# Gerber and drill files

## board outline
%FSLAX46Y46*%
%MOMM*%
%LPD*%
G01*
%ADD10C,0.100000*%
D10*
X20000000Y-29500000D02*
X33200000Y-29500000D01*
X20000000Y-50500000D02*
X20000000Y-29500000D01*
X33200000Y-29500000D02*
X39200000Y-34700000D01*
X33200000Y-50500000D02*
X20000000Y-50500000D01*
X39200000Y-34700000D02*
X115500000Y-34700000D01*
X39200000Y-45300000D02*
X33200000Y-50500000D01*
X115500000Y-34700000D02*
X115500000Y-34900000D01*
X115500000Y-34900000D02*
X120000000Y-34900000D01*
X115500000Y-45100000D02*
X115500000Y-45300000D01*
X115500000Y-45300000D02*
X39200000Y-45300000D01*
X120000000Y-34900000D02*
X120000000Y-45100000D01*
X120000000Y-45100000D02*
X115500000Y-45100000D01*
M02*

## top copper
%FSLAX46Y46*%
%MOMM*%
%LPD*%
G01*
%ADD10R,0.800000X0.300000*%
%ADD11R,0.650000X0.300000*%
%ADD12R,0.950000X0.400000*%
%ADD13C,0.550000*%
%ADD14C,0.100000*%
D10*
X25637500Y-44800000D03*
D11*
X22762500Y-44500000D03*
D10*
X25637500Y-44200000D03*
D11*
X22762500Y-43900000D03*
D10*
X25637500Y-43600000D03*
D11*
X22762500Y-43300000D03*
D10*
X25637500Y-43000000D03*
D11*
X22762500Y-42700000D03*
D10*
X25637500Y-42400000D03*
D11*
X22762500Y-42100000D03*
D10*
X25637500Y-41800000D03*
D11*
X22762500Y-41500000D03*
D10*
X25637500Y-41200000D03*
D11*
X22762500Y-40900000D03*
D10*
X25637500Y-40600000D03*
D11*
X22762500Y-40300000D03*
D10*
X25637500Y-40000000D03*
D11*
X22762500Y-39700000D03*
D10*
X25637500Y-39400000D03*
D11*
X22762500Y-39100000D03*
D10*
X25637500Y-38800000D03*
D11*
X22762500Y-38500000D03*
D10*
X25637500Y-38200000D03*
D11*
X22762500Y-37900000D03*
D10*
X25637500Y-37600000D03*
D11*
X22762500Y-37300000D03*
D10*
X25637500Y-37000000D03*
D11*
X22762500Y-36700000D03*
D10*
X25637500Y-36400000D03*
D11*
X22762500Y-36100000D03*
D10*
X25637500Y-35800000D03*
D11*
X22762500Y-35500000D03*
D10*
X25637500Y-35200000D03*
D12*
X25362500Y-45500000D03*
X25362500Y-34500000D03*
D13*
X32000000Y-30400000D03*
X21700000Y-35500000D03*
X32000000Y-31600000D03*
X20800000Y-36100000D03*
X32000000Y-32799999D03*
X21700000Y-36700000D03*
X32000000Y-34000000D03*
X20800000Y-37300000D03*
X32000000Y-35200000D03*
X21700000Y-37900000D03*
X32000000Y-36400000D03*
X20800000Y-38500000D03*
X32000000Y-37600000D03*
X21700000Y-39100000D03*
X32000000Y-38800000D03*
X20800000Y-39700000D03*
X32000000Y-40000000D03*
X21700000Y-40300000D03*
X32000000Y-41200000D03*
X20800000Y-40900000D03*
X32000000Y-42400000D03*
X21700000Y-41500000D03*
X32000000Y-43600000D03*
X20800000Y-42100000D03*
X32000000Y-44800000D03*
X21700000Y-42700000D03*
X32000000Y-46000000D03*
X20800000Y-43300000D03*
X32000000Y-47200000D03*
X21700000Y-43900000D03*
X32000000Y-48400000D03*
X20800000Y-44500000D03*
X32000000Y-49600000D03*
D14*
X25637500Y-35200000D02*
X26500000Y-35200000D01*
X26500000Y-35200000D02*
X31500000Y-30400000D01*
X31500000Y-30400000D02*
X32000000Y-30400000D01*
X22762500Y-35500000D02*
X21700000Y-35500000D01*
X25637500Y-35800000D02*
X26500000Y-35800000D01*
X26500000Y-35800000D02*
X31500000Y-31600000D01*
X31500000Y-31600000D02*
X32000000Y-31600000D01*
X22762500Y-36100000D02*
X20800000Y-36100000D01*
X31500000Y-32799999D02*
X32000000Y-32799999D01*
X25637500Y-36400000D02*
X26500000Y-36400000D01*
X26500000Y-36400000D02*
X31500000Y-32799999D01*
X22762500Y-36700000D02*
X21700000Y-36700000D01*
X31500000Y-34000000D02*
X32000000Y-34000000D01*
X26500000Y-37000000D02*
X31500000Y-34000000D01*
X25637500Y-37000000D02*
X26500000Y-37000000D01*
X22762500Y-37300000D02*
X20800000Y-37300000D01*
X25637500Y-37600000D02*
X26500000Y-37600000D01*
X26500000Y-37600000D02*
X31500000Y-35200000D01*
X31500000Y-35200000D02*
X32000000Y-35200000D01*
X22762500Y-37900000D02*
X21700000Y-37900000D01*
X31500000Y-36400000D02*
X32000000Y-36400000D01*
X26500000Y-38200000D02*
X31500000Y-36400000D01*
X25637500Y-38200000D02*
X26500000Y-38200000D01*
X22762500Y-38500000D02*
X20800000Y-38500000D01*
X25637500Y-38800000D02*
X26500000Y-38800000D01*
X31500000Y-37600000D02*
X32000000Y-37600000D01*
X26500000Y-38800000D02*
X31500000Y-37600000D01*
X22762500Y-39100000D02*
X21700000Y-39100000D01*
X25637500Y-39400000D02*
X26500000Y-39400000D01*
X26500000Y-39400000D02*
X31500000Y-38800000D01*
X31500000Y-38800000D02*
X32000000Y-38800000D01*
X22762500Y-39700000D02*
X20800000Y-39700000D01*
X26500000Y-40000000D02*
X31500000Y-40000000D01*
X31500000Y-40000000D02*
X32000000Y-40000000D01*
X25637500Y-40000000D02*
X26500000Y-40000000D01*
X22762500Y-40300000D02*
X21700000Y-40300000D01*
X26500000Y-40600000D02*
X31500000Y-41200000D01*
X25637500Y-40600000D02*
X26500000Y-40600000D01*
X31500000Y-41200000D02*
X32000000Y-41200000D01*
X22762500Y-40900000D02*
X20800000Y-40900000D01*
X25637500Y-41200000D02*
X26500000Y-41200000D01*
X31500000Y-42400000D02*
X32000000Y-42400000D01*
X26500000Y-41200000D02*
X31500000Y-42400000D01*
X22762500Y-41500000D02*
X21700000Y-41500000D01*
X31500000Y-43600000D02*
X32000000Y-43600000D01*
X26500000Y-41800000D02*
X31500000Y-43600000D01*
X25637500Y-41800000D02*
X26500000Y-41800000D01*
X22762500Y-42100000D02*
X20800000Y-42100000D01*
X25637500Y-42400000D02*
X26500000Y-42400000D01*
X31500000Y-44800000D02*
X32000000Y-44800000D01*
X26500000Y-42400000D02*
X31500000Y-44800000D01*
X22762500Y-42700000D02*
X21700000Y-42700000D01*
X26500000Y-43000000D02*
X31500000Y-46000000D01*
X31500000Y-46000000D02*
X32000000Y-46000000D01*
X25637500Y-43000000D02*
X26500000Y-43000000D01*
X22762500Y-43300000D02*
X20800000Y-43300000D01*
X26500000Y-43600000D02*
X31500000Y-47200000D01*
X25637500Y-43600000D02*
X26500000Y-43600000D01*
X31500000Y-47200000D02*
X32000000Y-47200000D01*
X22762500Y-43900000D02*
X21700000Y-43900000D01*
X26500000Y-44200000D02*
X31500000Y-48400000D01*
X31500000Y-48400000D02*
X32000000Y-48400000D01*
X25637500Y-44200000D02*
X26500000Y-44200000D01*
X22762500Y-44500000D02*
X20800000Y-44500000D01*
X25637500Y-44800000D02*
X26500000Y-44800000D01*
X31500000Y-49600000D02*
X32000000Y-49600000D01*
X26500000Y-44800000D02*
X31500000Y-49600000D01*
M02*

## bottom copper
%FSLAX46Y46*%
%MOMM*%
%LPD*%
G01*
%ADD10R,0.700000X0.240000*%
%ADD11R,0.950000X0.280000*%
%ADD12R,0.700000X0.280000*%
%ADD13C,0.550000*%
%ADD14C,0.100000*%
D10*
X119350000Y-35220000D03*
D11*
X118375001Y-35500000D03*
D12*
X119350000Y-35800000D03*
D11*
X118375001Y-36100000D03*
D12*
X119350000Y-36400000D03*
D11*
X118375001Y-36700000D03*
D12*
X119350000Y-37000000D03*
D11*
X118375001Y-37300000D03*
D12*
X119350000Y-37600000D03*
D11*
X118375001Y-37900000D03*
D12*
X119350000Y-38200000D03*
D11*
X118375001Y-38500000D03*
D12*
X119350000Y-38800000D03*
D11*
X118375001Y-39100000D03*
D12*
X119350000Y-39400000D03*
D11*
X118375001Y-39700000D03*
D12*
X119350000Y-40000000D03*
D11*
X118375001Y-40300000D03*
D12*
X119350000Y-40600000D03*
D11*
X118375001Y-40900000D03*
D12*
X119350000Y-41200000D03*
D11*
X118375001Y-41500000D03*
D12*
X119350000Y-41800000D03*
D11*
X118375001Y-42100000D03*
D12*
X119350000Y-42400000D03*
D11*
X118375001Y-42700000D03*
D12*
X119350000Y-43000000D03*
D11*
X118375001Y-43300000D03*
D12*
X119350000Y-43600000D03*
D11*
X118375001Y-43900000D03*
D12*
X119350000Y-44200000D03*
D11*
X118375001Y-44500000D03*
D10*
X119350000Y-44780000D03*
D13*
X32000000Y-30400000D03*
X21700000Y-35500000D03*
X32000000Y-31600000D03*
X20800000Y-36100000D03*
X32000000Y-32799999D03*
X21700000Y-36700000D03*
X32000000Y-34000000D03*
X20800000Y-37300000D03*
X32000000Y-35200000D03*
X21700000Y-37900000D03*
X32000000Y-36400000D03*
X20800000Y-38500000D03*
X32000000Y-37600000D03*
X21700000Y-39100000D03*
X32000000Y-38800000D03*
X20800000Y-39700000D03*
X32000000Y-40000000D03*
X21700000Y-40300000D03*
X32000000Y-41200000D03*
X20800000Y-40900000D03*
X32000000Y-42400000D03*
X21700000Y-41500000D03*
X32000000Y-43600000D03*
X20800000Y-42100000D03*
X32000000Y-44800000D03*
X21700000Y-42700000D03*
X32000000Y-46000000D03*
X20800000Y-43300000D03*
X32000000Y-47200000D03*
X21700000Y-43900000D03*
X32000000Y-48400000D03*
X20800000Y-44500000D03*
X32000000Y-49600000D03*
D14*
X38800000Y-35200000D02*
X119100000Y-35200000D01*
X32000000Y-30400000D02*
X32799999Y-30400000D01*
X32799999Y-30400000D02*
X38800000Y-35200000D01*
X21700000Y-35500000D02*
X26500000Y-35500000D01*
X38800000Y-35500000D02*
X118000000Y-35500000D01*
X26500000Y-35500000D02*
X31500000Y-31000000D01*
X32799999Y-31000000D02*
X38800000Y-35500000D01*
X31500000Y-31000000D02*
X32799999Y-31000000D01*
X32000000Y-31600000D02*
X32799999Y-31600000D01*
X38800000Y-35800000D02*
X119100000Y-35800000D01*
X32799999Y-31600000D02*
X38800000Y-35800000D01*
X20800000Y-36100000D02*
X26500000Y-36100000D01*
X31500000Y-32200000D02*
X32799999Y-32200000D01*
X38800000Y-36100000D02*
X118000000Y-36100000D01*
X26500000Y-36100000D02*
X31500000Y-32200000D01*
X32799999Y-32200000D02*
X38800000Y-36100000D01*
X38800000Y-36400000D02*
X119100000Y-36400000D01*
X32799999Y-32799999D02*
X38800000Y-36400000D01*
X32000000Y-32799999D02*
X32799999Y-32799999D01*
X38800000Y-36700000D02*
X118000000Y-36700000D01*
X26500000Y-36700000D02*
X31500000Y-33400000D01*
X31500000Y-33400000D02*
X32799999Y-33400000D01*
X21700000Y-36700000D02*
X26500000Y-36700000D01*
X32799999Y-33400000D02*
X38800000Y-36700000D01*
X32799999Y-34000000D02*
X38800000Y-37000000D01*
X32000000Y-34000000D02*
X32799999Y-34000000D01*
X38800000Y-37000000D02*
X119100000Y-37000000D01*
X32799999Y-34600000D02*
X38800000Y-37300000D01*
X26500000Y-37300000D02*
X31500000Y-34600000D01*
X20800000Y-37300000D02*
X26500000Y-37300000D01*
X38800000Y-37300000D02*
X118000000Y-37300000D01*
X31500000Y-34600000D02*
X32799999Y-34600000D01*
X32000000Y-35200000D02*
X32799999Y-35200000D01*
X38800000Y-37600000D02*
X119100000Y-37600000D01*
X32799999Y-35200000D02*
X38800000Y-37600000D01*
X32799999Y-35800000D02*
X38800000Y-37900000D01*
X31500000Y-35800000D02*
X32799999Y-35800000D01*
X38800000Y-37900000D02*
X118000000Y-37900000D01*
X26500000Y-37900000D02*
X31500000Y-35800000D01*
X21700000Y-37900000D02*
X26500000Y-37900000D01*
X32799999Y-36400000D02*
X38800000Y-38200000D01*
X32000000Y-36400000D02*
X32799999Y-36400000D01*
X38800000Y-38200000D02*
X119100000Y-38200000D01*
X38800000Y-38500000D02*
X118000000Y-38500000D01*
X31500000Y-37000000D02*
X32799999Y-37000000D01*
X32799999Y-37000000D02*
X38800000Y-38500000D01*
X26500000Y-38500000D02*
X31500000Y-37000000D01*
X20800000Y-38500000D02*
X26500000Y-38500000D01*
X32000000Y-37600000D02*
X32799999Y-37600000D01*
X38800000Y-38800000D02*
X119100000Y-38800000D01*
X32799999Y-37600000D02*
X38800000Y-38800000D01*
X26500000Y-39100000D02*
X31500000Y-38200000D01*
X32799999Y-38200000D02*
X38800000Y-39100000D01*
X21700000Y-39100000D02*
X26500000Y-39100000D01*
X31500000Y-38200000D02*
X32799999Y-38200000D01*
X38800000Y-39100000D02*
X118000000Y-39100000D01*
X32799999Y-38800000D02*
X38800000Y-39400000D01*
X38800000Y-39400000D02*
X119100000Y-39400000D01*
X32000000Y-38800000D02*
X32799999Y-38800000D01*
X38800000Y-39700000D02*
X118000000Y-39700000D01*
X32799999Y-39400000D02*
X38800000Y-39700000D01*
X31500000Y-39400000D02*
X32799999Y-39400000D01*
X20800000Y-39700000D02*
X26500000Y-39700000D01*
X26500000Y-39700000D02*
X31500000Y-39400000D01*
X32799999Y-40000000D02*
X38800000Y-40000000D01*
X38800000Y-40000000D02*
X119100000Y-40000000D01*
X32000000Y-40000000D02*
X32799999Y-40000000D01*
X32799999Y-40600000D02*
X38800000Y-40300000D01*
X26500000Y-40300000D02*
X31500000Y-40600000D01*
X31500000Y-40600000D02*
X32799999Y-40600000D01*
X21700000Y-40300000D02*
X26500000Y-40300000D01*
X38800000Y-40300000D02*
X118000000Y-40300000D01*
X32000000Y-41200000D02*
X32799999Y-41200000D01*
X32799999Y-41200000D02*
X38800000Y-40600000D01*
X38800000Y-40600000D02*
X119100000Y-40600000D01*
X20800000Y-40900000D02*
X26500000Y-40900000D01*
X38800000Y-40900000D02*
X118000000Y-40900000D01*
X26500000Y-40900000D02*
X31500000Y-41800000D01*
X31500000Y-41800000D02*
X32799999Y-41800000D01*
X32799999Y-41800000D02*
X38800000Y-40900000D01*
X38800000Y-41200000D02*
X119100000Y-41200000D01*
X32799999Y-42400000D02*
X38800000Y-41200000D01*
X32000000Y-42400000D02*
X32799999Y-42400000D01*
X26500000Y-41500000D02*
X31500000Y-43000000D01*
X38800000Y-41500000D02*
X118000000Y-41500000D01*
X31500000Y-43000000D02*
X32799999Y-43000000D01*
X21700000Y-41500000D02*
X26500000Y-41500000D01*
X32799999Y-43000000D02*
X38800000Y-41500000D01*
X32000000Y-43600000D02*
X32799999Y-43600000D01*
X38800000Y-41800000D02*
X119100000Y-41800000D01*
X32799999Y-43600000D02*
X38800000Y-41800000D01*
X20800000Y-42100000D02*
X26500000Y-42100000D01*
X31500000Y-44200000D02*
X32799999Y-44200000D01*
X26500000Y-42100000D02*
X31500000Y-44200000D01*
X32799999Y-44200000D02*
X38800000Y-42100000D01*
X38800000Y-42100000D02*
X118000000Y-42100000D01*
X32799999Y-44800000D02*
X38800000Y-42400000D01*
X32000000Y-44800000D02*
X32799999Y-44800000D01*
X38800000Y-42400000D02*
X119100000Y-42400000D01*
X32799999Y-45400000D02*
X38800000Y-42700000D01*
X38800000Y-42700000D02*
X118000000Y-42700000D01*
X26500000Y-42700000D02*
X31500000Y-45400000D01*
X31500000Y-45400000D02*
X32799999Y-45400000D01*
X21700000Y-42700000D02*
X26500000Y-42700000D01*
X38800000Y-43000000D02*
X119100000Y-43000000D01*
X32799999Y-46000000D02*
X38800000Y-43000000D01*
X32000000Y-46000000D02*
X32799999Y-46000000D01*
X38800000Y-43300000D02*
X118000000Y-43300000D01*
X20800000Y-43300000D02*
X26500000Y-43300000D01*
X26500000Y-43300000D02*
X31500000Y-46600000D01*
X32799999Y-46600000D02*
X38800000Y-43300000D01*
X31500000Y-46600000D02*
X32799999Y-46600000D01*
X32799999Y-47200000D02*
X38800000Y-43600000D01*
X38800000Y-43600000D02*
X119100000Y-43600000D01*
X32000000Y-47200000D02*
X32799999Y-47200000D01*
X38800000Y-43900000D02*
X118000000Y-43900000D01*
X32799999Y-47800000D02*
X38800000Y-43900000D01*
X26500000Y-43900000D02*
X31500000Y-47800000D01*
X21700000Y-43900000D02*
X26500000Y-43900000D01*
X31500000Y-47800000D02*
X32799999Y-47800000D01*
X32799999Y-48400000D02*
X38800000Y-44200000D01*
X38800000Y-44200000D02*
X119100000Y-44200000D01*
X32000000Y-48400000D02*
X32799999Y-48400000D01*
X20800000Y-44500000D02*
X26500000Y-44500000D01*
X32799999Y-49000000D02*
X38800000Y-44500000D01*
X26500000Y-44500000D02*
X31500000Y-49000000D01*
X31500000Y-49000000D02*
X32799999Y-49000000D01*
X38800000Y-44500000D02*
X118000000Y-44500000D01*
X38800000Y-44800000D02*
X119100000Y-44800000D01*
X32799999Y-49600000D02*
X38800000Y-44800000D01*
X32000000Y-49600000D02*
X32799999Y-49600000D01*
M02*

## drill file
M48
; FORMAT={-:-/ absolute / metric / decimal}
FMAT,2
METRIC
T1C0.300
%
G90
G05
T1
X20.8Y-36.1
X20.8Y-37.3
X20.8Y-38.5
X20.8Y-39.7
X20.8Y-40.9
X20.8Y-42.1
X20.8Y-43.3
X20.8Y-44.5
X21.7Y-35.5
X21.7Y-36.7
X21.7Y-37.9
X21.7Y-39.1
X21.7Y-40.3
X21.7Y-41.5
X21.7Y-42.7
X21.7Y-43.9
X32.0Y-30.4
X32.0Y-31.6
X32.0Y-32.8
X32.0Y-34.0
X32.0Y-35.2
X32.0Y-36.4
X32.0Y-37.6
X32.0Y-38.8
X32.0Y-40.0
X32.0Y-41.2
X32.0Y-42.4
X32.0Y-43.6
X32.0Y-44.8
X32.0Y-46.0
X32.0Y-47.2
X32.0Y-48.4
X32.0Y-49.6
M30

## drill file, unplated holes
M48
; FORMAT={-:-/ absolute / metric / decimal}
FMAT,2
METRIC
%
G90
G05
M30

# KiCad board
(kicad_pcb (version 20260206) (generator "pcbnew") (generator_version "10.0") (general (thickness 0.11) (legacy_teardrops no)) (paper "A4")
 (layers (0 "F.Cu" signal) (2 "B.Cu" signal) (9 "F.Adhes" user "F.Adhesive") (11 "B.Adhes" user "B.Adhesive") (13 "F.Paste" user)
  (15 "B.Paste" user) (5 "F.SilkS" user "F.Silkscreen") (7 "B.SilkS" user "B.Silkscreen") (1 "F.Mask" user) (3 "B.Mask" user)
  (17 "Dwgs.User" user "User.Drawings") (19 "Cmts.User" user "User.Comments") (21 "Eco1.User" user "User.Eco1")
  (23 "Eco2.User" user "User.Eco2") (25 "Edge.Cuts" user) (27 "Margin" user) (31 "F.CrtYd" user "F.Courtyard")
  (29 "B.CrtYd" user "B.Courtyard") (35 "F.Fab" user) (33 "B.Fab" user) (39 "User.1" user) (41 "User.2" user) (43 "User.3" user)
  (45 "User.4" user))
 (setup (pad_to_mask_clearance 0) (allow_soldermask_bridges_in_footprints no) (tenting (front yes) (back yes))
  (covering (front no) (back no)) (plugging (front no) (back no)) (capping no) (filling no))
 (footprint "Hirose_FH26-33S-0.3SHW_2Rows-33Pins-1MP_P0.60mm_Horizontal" (layer "F.Cu") (at 24.2375 40 180)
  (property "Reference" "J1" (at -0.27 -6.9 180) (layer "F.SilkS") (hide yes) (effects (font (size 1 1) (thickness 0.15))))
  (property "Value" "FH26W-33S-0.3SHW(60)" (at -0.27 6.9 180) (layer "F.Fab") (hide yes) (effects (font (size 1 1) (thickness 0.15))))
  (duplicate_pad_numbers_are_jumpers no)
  (pad "1" smd rect (at -1.4 -4.8 180) (size 0.8 0.3) (layers "F.Cu" "F.Mask" "F.Paste") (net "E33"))
  (pad "2" smd rect (at 1.475 -4.5 180) (size 0.65 0.3) (layers "F.Cu" "F.Mask" "F.Paste") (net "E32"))
  (pad "3" smd rect (at -1.4 -4.2 180) (size 0.8 0.3) (layers "F.Cu" "F.Mask" "F.Paste") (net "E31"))
  (pad "4" smd rect (at 1.475 -3.9 180) (size 0.65 0.3) (layers "F.Cu" "F.Mask" "F.Paste") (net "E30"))
  (pad "5" smd rect (at -1.4 -3.6 180) (size 0.8 0.3) (layers "F.Cu" "F.Mask" "F.Paste") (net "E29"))
  (pad "6" smd rect (at 1.475 -3.3 180) (size 0.65 0.3) (layers "F.Cu" "F.Mask" "F.Paste") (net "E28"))
  (pad "7" smd rect (at -1.4 -3 180) (size 0.8 0.3) (layers "F.Cu" "F.Mask" "F.Paste") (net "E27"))
  (pad "8" smd rect (at 1.475 -2.7 180) (size 0.65 0.3) (layers "F.Cu" "F.Mask" "F.Paste") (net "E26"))
  (pad "9" smd rect (at -1.4 -2.4 180) (size 0.8 0.3) (layers "F.Cu" "F.Mask" "F.Paste") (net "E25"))
  (pad "10" smd rect (at 1.475 -2.1 180) (size 0.65 0.3) (layers "F.Cu" "F.Mask" "F.Paste") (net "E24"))
  (pad "11" smd rect (at -1.4 -1.8 180) (size 0.8 0.3) (layers "F.Cu" "F.Mask" "F.Paste") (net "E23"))
  (pad "12" smd rect (at 1.475 -1.5 180) (size 0.65 0.3) (layers "F.Cu" "F.Mask" "F.Paste") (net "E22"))
  (pad "13" smd rect (at -1.4 -1.2 180) (size 0.8 0.3) (layers "F.Cu" "F.Mask" "F.Paste") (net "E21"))
  (pad "14" smd rect (at 1.475 -0.9 180) (size 0.65 0.3) (layers "F.Cu" "F.Mask" "F.Paste") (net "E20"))
  (pad "15" smd rect (at -1.4 -0.6 180) (size 0.8 0.3) (layers "F.Cu" "F.Mask" "F.Paste") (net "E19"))
  (pad "16" smd rect (at 1.475 -0.3 180) (size 0.65 0.3) (layers "F.Cu" "F.Mask" "F.Paste") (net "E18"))
  (pad "17" smd rect (at -1.4 0 180) (size 0.8 0.3) (layers "F.Cu" "F.Mask" "F.Paste") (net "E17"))
  (pad "18" smd rect (at 1.475 0.3 180) (size 0.65 0.3) (layers "F.Cu" "F.Mask" "F.Paste") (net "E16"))
  (pad "19" smd rect (at -1.4 0.6 180) (size 0.8 0.3) (layers "F.Cu" "F.Mask" "F.Paste") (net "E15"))
  (pad "20" smd rect (at 1.475 0.9 180) (size 0.65 0.3) (layers "F.Cu" "F.Mask" "F.Paste") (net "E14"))
  (pad "21" smd rect (at -1.4 1.2 180) (size 0.8 0.3) (layers "F.Cu" "F.Mask" "F.Paste") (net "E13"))
  (pad "22" smd rect (at 1.475 1.5 180) (size 0.65 0.3) (layers "F.Cu" "F.Mask" "F.Paste") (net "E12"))
  (pad "23" smd rect (at -1.4 1.8 180) (size 0.8 0.3) (layers "F.Cu" "F.Mask" "F.Paste") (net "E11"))
  (pad "24" smd rect (at 1.475 2.1 180) (size 0.65 0.3) (layers "F.Cu" "F.Mask" "F.Paste") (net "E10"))
  (pad "25" smd rect (at -1.4 2.4 180) (size 0.8 0.3) (layers "F.Cu" "F.Mask" "F.Paste") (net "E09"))
  (pad "26" smd rect (at 1.475 2.7 180) (size 0.65 0.3) (layers "F.Cu" "F.Mask" "F.Paste") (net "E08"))
  (pad "27" smd rect (at -1.4 3 180) (size 0.8 0.3) (layers "F.Cu" "F.Mask" "F.Paste") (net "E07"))
  (pad "28" smd rect (at 1.475 3.3 180) (size 0.65 0.3) (layers "F.Cu" "F.Mask" "F.Paste") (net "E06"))
  (pad "29" smd rect (at -1.4 3.6 180) (size 0.8 0.3) (layers "F.Cu" "F.Mask" "F.Paste") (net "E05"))
  (pad "30" smd rect (at 1.475 3.9 180) (size 0.65 0.3) (layers "F.Cu" "F.Mask" "F.Paste") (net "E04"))
  (pad "31" smd rect (at -1.4 4.2 180) (size 0.8 0.3) (layers "F.Cu" "F.Mask" "F.Paste") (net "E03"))
  (pad "32" smd rect (at 1.475 4.5 180) (size 0.65 0.3) (layers "F.Cu" "F.Mask" "F.Paste") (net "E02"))
  (pad "33" smd rect (at -1.4 4.8 180) (size 0.8 0.3) (layers "F.Cu" "F.Mask" "F.Paste") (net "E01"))
  (pad "MP" smd rect (at -1.125 -5.5 180) (size 0.95 0.4) (layers "F.Cu" "F.Mask" "F.Paste"))
  (pad "MP" smd rect (at -1.125 5.5 180) (size 0.95 0.4) (layers "F.Cu" "F.Mask" "F.Paste")))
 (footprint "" (layer "B.Cu") (at 118.6 40 180)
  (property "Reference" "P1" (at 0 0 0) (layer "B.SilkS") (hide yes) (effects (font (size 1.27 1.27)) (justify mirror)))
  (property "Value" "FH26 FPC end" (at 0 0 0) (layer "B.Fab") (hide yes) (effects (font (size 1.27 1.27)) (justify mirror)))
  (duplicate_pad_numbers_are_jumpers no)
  (pad "1" smd rect (at -0.75 4.78 180) (size 0.7 0.24) (layers "B.Cu" "B.Mask") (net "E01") (thermal_bridge_angle 45))
  (pad "2" smd rect (at 0.224999 4.5 180) (size 0.95 0.28) (layers "B.Cu" "B.Mask") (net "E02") (thermal_bridge_angle 45))
  (pad "3" smd rect (at -0.75 4.2 180) (size 0.7 0.28) (layers "B.Cu" "B.Mask") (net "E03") (thermal_bridge_angle 45))
  (pad "4" smd rect (at 0.224999 3.9 180) (size 0.95 0.28) (layers "B.Cu" "B.Mask") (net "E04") (thermal_bridge_angle 45))
  (pad "5" smd rect (at -0.75 3.6 180) (size 0.7 0.28) (layers "B.Cu" "B.Mask") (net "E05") (thermal_bridge_angle 45))
  (pad "6" smd rect (at 0.224999 3.3 180) (size 0.95 0.28) (layers "B.Cu" "B.Mask") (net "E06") (thermal_bridge_angle 45))
  (pad "7" smd rect (at -0.75 3 180) (size 0.7 0.28) (layers "B.Cu" "B.Mask") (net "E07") (thermal_bridge_angle 45))
  (pad "8" smd rect (at 0.224999 2.7 180) (size 0.95 0.28) (layers "B.Cu" "B.Mask") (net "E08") (thermal_bridge_angle 45))
  (pad "9" smd rect (at -0.75 2.4 180) (size 0.7 0.28) (layers "B.Cu" "B.Mask") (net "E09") (thermal_bridge_angle 45))
  (pad "10" smd rect (at 0.224999 2.1 180) (size 0.95 0.28) (layers "B.Cu" "B.Mask") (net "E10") (thermal_bridge_angle 45))
  (pad "11" smd rect (at -0.75 1.8 180) (size 0.7 0.28) (layers "B.Cu" "B.Mask") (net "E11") (thermal_bridge_angle 45))
  (pad "12" smd rect (at 0.224999 1.5 180) (size 0.95 0.28) (layers "B.Cu" "B.Mask") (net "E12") (thermal_bridge_angle 45))
  (pad "13" smd rect (at -0.75 1.2 180) (size 0.7 0.28) (layers "B.Cu" "B.Mask") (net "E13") (thermal_bridge_angle 45))
  (pad "14" smd rect (at 0.224999 0.9 180) (size 0.95 0.28) (layers "B.Cu" "B.Mask") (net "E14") (thermal_bridge_angle 45))
  (pad "15" smd rect (at -0.75 0.6 180) (size 0.7 0.28) (layers "B.Cu" "B.Mask") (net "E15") (thermal_bridge_angle 45))
  (pad "16" smd rect (at 0.224999 0.3 180) (size 0.95 0.28) (layers "B.Cu" "B.Mask") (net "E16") (thermal_bridge_angle 45))
  (pad "17" smd rect (at -0.75 0 180) (size 0.7 0.28) (layers "B.Cu" "B.Mask") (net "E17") (thermal_bridge_angle 45))
  (pad "18" smd rect (at 0.224999 -0.3 180) (size 0.95 0.28) (layers "B.Cu" "B.Mask") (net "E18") (thermal_bridge_angle 45))
  (pad "19" smd rect (at -0.75 -0.6 180) (size 0.7 0.28) (layers "B.Cu" "B.Mask") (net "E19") (thermal_bridge_angle 45))
  (pad "20" smd rect (at 0.224999 -0.9 180) (size 0.95 0.28) (layers "B.Cu" "B.Mask") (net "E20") (thermal_bridge_angle 45))
  (pad "21" smd rect (at -0.75 -1.2 180) (size 0.7 0.28) (layers "B.Cu" "B.Mask") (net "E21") (thermal_bridge_angle 45))
  (pad "22" smd rect (at 0.224999 -1.5 180) (size 0.95 0.28) (layers "B.Cu" "B.Mask") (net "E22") (thermal_bridge_angle 45))
  (pad "23" smd rect (at -0.75 -1.8 180) (size 0.7 0.28) (layers "B.Cu" "B.Mask") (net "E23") (thermal_bridge_angle 45))
  (pad "24" smd rect (at 0.224999 -2.1 180) (size 0.95 0.28) (layers "B.Cu" "B.Mask") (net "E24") (thermal_bridge_angle 45))
  (pad "25" smd rect (at -0.75 -2.4 180) (size 0.7 0.28) (layers "B.Cu" "B.Mask") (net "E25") (thermal_bridge_angle 45))
  (pad "26" smd rect (at 0.224999 -2.7 180) (size 0.95 0.28) (layers "B.Cu" "B.Mask") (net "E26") (thermal_bridge_angle 45))
  (pad "27" smd rect (at -0.75 -3 180) (size 0.7 0.28) (layers "B.Cu" "B.Mask") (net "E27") (thermal_bridge_angle 45))
  (pad "28" smd rect (at 0.224999 -3.3 180) (size 0.95 0.28) (layers "B.Cu" "B.Mask") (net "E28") (thermal_bridge_angle 45))
  (pad "29" smd rect (at -0.75 -3.6 180) (size 0.7 0.28) (layers "B.Cu" "B.Mask") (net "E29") (thermal_bridge_angle 45))
  (pad "30" smd rect (at 0.224999 -3.9 180) (size 0.95 0.28) (layers "B.Cu" "B.Mask") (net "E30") (thermal_bridge_angle 45))
  (pad "31" smd rect (at -0.75 -4.2 180) (size 0.7 0.28) (layers "B.Cu" "B.Mask") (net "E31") (thermal_bridge_angle 45))
  (pad "32" smd rect (at 0.224999 -4.5 180) (size 0.95 0.28) (layers "B.Cu" "B.Mask") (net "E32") (thermal_bridge_angle 45))
  (pad "33" smd rect (at -0.75 -4.78 180) (size 0.7 0.24) (layers "B.Cu" "B.Mask") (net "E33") (thermal_bridge_angle 45)))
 (gr_line (start 20 29.5) (end 33.2 29.5) (stroke (width 0.1) (type default)) (layer "Edge.Cuts"))
 (gr_line (start 20 50.5) (end 20 29.5) (stroke (width 0.1) (type default)) (layer "Edge.Cuts"))
 (gr_line (start 33.2 29.5) (end 39.2 34.7) (stroke (width 0.1) (type default)) (layer "Edge.Cuts"))
 (gr_line (start 33.2 50.5) (end 20 50.5) (stroke (width 0.1) (type default)) (layer "Edge.Cuts"))
 (gr_line (start 39.2 34.7) (end 115.5 34.7) (stroke (width 0.1) (type default)) (layer "Edge.Cuts"))
 (gr_line (start 39.2 45.3) (end 33.2 50.5) (stroke (width 0.1) (type default)) (layer "Edge.Cuts"))
 (gr_line (start 115.5 34.7) (end 115.5 34.9) (stroke (width 0.1) (type default)) (layer "Edge.Cuts"))
 (gr_line (start 115.5 34.9) (end 120 34.9) (stroke (width 0.1) (type default)) (layer "Edge.Cuts"))
 (gr_line (start 115.5 45.1) (end 115.5 45.3) (stroke (width 0.1) (type default)) (layer "Edge.Cuts"))
 (gr_line (start 115.5 45.3) (end 39.2 45.3) (stroke (width 0.1) (type default)) (layer "Edge.Cuts"))
 (gr_line (start 120 34.9) (end 120 45.1) (stroke (width 0.1) (type default)) (layer "Edge.Cuts"))
 (gr_line (start 120 45.1) (end 115.5 45.1) (stroke (width 0.1) (type default)) (layer "Edge.Cuts"))
 (segment (start 25.6375 35.2) (end 26.5 35.2) (width 0.1) (layer "F.Cu") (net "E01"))
 (segment (start 26.5 35.2) (end 31.5 30.4) (width 0.1) (layer "F.Cu") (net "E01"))
 (segment (start 31.5 30.4) (end 32 30.4) (width 0.1) (layer "F.Cu") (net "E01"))
 (via (at 32 30.4) (size 0.55) (drill 0.3) (layers "F.Cu" "B.Cu") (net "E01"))
 (segment (start 38.8 35.2) (end 119.1 35.2) (width 0.1) (layer "B.Cu") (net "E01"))
 (segment (start 32 30.4) (end 32.799999 30.4) (width 0.1) (layer "B.Cu") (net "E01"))
 (segment (start 32.799999 30.4) (end 38.8 35.2) (width 0.1) (layer "B.Cu") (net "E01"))
 (segment (start 22.7625 35.5) (end 21.7 35.5) (width 0.1) (layer "F.Cu") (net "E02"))
 (via (at 21.7 35.5) (size 0.55) (drill 0.3) (layers "F.Cu" "B.Cu") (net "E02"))
 (segment (start 21.7 35.5) (end 26.5 35.5) (width 0.1) (layer "B.Cu") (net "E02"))
 (segment (start 38.8 35.5) (end 118 35.5) (width 0.1) (layer "B.Cu") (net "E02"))
 (segment (start 26.5 35.5) (end 31.5 31) (width 0.1) (layer "B.Cu") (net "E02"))
 (segment (start 32.799999 31) (end 38.8 35.5) (width 0.1) (layer "B.Cu") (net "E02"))
 (segment (start 31.5 31) (end 32.799999 31) (width 0.1) (layer "B.Cu") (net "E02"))
 (segment (start 25.6375 35.8) (end 26.5 35.8) (width 0.1) (layer "F.Cu") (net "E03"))
 (segment (start 26.5 35.8) (end 31.5 31.6) (width 0.1) (layer "F.Cu") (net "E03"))
 (segment (start 31.5 31.6) (end 32 31.6) (width 0.1) (layer "F.Cu") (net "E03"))
 (via (at 32 31.6) (size 0.55) (drill 0.3) (layers "F.Cu" "B.Cu") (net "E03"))
 (segment (start 32 31.6) (end 32.799999 31.6) (width 0.1) (layer "B.Cu") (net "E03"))
 (segment (start 38.8 35.8) (end 119.1 35.8) (width 0.1) (layer "B.Cu") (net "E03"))
 (segment (start 32.799999 31.6) (end 38.8 35.8) (width 0.1) (layer "B.Cu") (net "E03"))
 (segment (start 22.7625 36.1) (end 20.8 36.1) (width 0.1) (layer "F.Cu") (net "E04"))
 (via (at 20.8 36.1) (size 0.55) (drill 0.3) (layers "F.Cu" "B.Cu") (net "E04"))
 (segment (start 20.8 36.1) (end 26.5 36.1) (width 0.1) (layer "B.Cu") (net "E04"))
 (segment (start 31.5 32.2) (end 32.799999 32.2) (width 0.1) (layer "B.Cu") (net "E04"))
 (segment (start 38.8 36.1) (end 118 36.1) (width 0.1) (layer "B.Cu") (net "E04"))
 (segment (start 26.5 36.1) (end 31.5 32.2) (width 0.1) (layer "B.Cu") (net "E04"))
 (segment (start 32.799999 32.2) (end 38.8 36.1) (width 0.1) (layer "B.Cu") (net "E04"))
 (segment (start 31.5 32.799999) (end 32 32.799999) (width 0.1) (layer "F.Cu") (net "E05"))
 (segment (start 25.6375 36.4) (end 26.5 36.4) (width 0.1) (layer "F.Cu") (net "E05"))
 (segment (start 26.5 36.4) (end 31.5 32.799999) (width 0.1) (layer "F.Cu") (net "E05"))
 (via (at 32 32.799999) (size 0.55) (drill 0.3) (layers "F.Cu" "B.Cu") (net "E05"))
 (segment (start 38.8 36.4) (end 119.1 36.4) (width 0.1) (layer "B.Cu") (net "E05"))
 (segment (start 32.799999 32.799999) (end 38.8 36.4) (width 0.1) (layer "B.Cu") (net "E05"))
 (segment (start 32 32.799999) (end 32.799999 32.799999) (width 0.1) (layer "B.Cu") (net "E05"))
 (segment (start 22.7625 36.7) (end 21.7 36.7) (width 0.1) (layer "F.Cu") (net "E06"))
 (via (at 21.7 36.7) (size 0.55) (drill 0.3) (layers "F.Cu" "B.Cu") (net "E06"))
 (segment (start 38.8 36.7) (end 118 36.7) (width 0.1) (layer "B.Cu") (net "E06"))
 (segment (start 26.5 36.7) (end 31.5 33.4) (width 0.1) (layer "B.Cu") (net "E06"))
 (segment (start 31.5 33.4) (end 32.799999 33.4) (width 0.1) (layer "B.Cu") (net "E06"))
 (segment (start 21.7 36.7) (end 26.5 36.7) (width 0.1) (layer "B.Cu") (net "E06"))
 (segment (start 32.799999 33.4) (end 38.8 36.7) (width 0.1) (layer "B.Cu") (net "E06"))
 (segment (start 31.5 34) (end 32 34) (width 0.1) (layer "F.Cu") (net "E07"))
 (segment (start 26.5 37) (end 31.5 34) (width 0.1) (layer "F.Cu") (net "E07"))
 (segment (start 25.6375 37) (end 26.5 37) (width 0.1) (layer "F.Cu") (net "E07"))
 (via (at 32 34) (size 0.55) (drill 0.3) (layers "F.Cu" "B.Cu") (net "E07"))
 (segment (start 32.799999 34) (end 38.8 37) (width 0.1) (layer "B.Cu") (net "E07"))
 (segment (start 32 34) (end 32.799999 34) (width 0.1) (layer "B.Cu") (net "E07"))
 (segment (start 38.8 37) (end 119.1 37) (width 0.1) (layer "B.Cu") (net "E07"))
 (segment (start 22.7625 37.3) (end 20.8 37.3) (width 0.1) (layer "F.Cu") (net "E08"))
 (via (at 20.8 37.3) (size 0.55) (drill 0.3) (layers "F.Cu" "B.Cu") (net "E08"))
 (segment (start 32.799999 34.6) (end 38.8 37.3) (width 0.1) (layer "B.Cu") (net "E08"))
 (segment (start 26.5 37.3) (end 31.5 34.6) (width 0.1) (layer "B.Cu") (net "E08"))
 (segment (start 20.8 37.3) (end 26.5 37.3) (width 0.1) (layer "B.Cu") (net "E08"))
 (segment (start 38.8 37.3) (end 118 37.3) (width 0.1) (layer "B.Cu") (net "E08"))
 (segment (start 31.5 34.6) (end 32.799999 34.6) (width 0.1) (layer "B.Cu") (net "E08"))
 (segment (start 25.6375 37.6) (end 26.5 37.6) (width 0.1) (layer "F.Cu") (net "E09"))
 (segment (start 26.5 37.6) (end 31.5 35.2) (width 0.1) (layer "F.Cu") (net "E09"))
 (segment (start 31.5 35.2) (end 32 35.2) (width 0.1) (layer "F.Cu") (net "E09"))
 (via (at 32 35.2) (size 0.55) (drill 0.3) (layers "F.Cu" "B.Cu") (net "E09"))
 (segment (start 32 35.2) (end 32.799999 35.2) (width 0.1) (layer "B.Cu") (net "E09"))
 (segment (start 38.8 37.6) (end 119.1 37.6) (width 0.1) (layer "B.Cu") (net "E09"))
 (segment (start 32.799999 35.2) (end 38.8 37.6) (width 0.1) (layer "B.Cu") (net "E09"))
 (segment (start 22.7625 37.9) (end 21.7 37.9) (width 0.1) (layer "F.Cu") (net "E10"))
 (via (at 21.7 37.9) (size 0.55) (drill 0.3) (layers "F.Cu" "B.Cu") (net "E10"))
 (segment (start 32.799999 35.8) (end 38.8 37.9) (width 0.1) (layer "B.Cu") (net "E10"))
 (segment (start 31.5 35.8) (end 32.799999 35.8) (width 0.1) (layer "B.Cu") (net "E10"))
 (segment (start 38.8 37.9) (end 118 37.9) (width 0.1) (layer "B.Cu") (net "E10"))
 (segment (start 26.5 37.9) (end 31.5 35.8) (width 0.1) (layer "B.Cu") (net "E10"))
 (segment (start 21.7 37.9) (end 26.5 37.9) (width 0.1) (layer "B.Cu") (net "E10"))
 (segment (start 31.5 36.4) (end 32 36.4) (width 0.1) (layer "F.Cu") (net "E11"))
 (segment (start 26.5 38.2) (end 31.5 36.4) (width 0.1) (layer "F.Cu") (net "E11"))
 (segment (start 25.6375 38.2) (end 26.5 38.2) (width 0.1) (layer "F.Cu") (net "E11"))
 (via (at 32 36.4) (size 0.55) (drill 0.3) (layers "F.Cu" "B.Cu") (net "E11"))
 (segment (start 32.799999 36.4) (end 38.8 38.2) (width 0.1) (layer "B.Cu") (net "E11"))
 (segment (start 32 36.4) (end 32.799999 36.4) (width 0.1) (layer "B.Cu") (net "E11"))
 (segment (start 38.8 38.2) (end 119.1 38.2) (width 0.1) (layer "B.Cu") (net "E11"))
 (segment (start 22.7625 38.5) (end 20.8 38.5) (width 0.1) (layer "F.Cu") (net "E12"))
 (via (at 20.8 38.5) (size 0.55) (drill 0.3) (layers "F.Cu" "B.Cu") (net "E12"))
 (segment (start 38.8 38.5) (end 118 38.5) (width 0.1) (layer "B.Cu") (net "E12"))
 (segment (start 31.5 37) (end 32.799999 37) (width 0.1) (layer "B.Cu") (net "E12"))
 (segment (start 32.799999 37) (end 38.8 38.5) (width 0.1) (layer "B.Cu") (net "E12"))
 (segment (start 26.5 38.5) (end 31.5 37) (width 0.1) (layer "B.Cu") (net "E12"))
 (segment (start 20.8 38.5) (end 26.5 38.5) (width 0.1) (layer "B.Cu") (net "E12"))
 (segment (start 25.6375 38.8) (end 26.5 38.8) (width 0.1) (layer "F.Cu") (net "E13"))
 (segment (start 31.5 37.6) (end 32 37.6) (width 0.1) (layer "F.Cu") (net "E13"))
 (segment (start 26.5 38.8) (end 31.5 37.6) (width 0.1) (layer "F.Cu") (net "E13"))
 (via (at 32 37.6) (size 0.55) (drill 0.3) (layers "F.Cu" "B.Cu") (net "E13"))
 (segment (start 32 37.6) (end 32.799999 37.6) (width 0.1) (layer "B.Cu") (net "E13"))
 (segment (start 38.8 38.8) (end 119.1 38.8) (width 0.1) (layer "B.Cu") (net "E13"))
 (segment (start 32.799999 37.6) (end 38.8 38.8) (width 0.1) (layer "B.Cu") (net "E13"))
 (segment (start 22.7625 39.1) (end 21.7 39.1) (width 0.1) (layer "F.Cu") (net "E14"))
 (via (at 21.7 39.1) (size 0.55) (drill 0.3) (layers "F.Cu" "B.Cu") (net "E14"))
 (segment (start 26.5 39.1) (end 31.5 38.2) (width 0.1) (layer "B.Cu") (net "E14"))
 (segment (start 32.799999 38.2) (end 38.8 39.1) (width 0.1) (layer "B.Cu") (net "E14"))
 (segment (start 21.7 39.1) (end 26.5 39.1) (width 0.1) (layer "B.Cu") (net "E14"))
 (segment (start 31.5 38.2) (end 32.799999 38.2) (width 0.1) (layer "B.Cu") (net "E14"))
 (segment (start 38.8 39.1) (end 118 39.1) (width 0.1) (layer "B.Cu") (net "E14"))
 (segment (start 25.6375 39.4) (end 26.5 39.4) (width 0.1) (layer "F.Cu") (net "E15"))
 (segment (start 26.5 39.4) (end 31.5 38.8) (width 0.1) (layer "F.Cu") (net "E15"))
 (segment (start 31.5 38.8) (end 32 38.8) (width 0.1) (layer "F.Cu") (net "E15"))
 (via (at 32 38.8) (size 0.55) (drill 0.3) (layers "F.Cu" "B.Cu") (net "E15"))
 (segment (start 32.799999 38.8) (end 38.8 39.4) (width 0.1) (layer "B.Cu") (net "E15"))
 (segment (start 38.8 39.4) (end 119.1 39.4) (width 0.1) (layer "B.Cu") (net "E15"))
 (segment (start 32 38.8) (end 32.799999 38.8) (width 0.1) (layer "B.Cu") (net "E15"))
 (segment (start 22.7625 39.7) (end 20.8 39.7) (width 0.1) (layer "F.Cu") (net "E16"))
 (via (at 20.8 39.7) (size 0.55) (drill 0.3) (layers "F.Cu" "B.Cu") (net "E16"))
 (segment (start 38.8 39.7) (end 118 39.7) (width 0.1) (layer "B.Cu") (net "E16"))
 (segment (start 32.799999 39.4) (end 38.8 39.7) (width 0.1) (layer "B.Cu") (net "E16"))
 (segment (start 31.5 39.4) (end 32.799999 39.4) (width 0.1) (layer "B.Cu") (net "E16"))
 (segment (start 20.8 39.7) (end 26.5 39.7) (width 0.1) (layer "B.Cu") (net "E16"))
 (segment (start 26.5 39.7) (end 31.5 39.4) (width 0.1) (layer "B.Cu") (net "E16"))
 (segment (start 26.5 40) (end 31.5 40) (width 0.1) (layer "F.Cu") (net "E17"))
 (segment (start 31.5 40) (end 32 40) (width 0.1) (layer "F.Cu") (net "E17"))
 (segment (start 25.6375 40) (end 26.5 40) (width 0.1) (layer "F.Cu") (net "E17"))
 (via (at 32 40) (size 0.55) (drill 0.3) (layers "F.Cu" "B.Cu") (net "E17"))
 (segment (start 32.799999 40) (end 38.8 40) (width 0.1) (layer "B.Cu") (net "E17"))
 (segment (start 38.8 40) (end 119.1 40) (width 0.1) (layer "B.Cu") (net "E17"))
 (segment (start 32 40) (end 32.799999 40) (width 0.1) (layer "B.Cu") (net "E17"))
 (segment (start 22.7625 40.3) (end 21.7 40.3) (width 0.1) (layer "F.Cu") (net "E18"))
 (via (at 21.7 40.3) (size 0.55) (drill 0.3) (layers "F.Cu" "B.Cu") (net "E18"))
 (segment (start 32.799999 40.6) (end 38.8 40.3) (width 0.1) (layer "B.Cu") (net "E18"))
 (segment (start 26.5 40.3) (end 31.5 40.6) (width 0.1) (layer "B.Cu") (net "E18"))
 (segment (start 31.5 40.6) (end 32.799999 40.6) (width 0.1) (layer "B.Cu") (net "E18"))
 (segment (start 21.7 40.3) (end 26.5 40.3) (width 0.1) (layer "B.Cu") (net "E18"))
 (segment (start 38.8 40.3) (end 118 40.3) (width 0.1) (layer "B.Cu") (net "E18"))
 (segment (start 26.5 40.6) (end 31.5 41.2) (width 0.1) (layer "F.Cu") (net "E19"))
 (segment (start 25.6375 40.6) (end 26.5 40.6) (width 0.1) (layer "F.Cu") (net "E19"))
 (segment (start 31.5 41.2) (end 32 41.2) (width 0.1) (layer "F.Cu") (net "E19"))
 (via (at 32 41.2) (size 0.55) (drill 0.3) (layers "F.Cu" "B.Cu") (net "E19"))
 (segment (start 32 41.2) (end 32.799999 41.2) (width 0.1) (layer "B.Cu") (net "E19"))
 (segment (start 32.799999 41.2) (end 38.8 40.6) (width 0.1) (layer "B.Cu") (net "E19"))
 (segment (start 38.8 40.6) (end 119.1 40.6) (width 0.1) (layer "B.Cu") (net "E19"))
 (segment (start 22.7625 40.9) (end 20.8 40.9) (width 0.1) (layer "F.Cu") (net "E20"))
 (via (at 20.8 40.9) (size 0.55) (drill 0.3) (layers "F.Cu" "B.Cu") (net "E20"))
 (segment (start 20.8 40.9) (end 26.5 40.9) (width 0.1) (layer "B.Cu") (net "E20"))
 (segment (start 38.8 40.9) (end 118 40.9) (width 0.1) (layer "B.Cu") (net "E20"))
 (segment (start 26.5 40.9) (end 31.5 41.8) (width 0.1) (layer "B.Cu") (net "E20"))
 (segment (start 31.5 41.8) (end 32.799999 41.8) (width 0.1) (layer "B.Cu") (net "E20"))
 (segment (start 32.799999 41.8) (end 38.8 40.9) (width 0.1) (layer "B.Cu") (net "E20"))
 (segment (start 25.6375 41.2) (end 26.5 41.2) (width 0.1) (layer "F.Cu") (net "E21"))
 (segment (start 31.5 42.4) (end 32 42.4) (width 0.1) (layer "F.Cu") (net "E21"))
 (segment (start 26.5 41.2) (end 31.5 42.4) (width 0.1) (layer "F.Cu") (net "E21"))
 (via (at 32 42.4) (size 0.55) (drill 0.3) (layers "F.Cu" "B.Cu") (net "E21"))
 (segment (start 38.8 41.2) (end 119.1 41.2) (width 0.1) (layer "B.Cu") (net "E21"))
 (segment (start 32.799999 42.4) (end 38.8 41.2) (width 0.1) (layer "B.Cu") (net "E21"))
 (segment (start 32 42.4) (end 32.799999 42.4) (width 0.1) (layer "B.Cu") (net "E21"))
 (segment (start 22.7625 41.5) (end 21.7 41.5) (width 0.1) (layer "F.Cu") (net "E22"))
 (via (at 21.7 41.5) (size 0.55) (drill 0.3) (layers "F.Cu" "B.Cu") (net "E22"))
 (segment (start 26.5 41.5) (end 31.5 43) (width 0.1) (layer "B.Cu") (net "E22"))
 (segment (start 38.8 41.5) (end 118 41.5) (width 0.1) (layer "B.Cu") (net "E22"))
 (segment (start 31.5 43) (end 32.799999 43) (width 0.1) (layer "B.Cu") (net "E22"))
 (segment (start 21.7 41.5) (end 26.5 41.5) (width 0.1) (layer "B.Cu") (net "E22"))
 (segment (start 32.799999 43) (end 38.8 41.5) (width 0.1) (layer "B.Cu") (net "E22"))
 (segment (start 31.5 43.6) (end 32 43.6) (width 0.1) (layer "F.Cu") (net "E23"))
 (segment (start 26.5 41.8) (end 31.5 43.6) (width 0.1) (layer "F.Cu") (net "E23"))
 (segment (start 25.6375 41.8) (end 26.5 41.8) (width 0.1) (layer "F.Cu") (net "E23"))
 (via (at 32 43.6) (size 0.55) (drill 0.3) (layers "F.Cu" "B.Cu") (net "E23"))
 (segment (start 32 43.6) (end 32.799999 43.6) (width 0.1) (layer "B.Cu") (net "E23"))
 (segment (start 38.8 41.8) (end 119.1 41.8) (width 0.1) (layer "B.Cu") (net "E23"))
 (segment (start 32.799999 43.6) (end 38.8 41.8) (width 0.1) (layer "B.Cu") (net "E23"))
 (segment (start 22.7625 42.1) (end 20.8 42.1) (width 0.1) (layer "F.Cu") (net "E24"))
 (via (at 20.8 42.1) (size 0.55) (drill 0.3) (layers "F.Cu" "B.Cu") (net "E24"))
 (segment (start 20.8 42.1) (end 26.5 42.1) (width 0.1) (layer "B.Cu") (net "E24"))
 (segment (start 31.5 44.2) (end 32.799999 44.2) (width 0.1) (layer "B.Cu") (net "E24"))
 (segment (start 26.5 42.1) (end 31.5 44.2) (width 0.1) (layer "B.Cu") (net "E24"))
 (segment (start 32.799999 44.2) (end 38.8 42.1) (width 0.1) (layer "B.Cu") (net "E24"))
 (segment (start 38.8 42.1) (end 118 42.1) (width 0.1) (layer "B.Cu") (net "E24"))
 (segment (start 25.6375 42.4) (end 26.5 42.4) (width 0.1) (layer "F.Cu") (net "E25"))
 (segment (start 31.5 44.8) (end 32 44.8) (width 0.1) (layer "F.Cu") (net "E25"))
 (segment (start 26.5 42.4) (end 31.5 44.8) (width 0.1) (layer "F.Cu") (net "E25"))
 (via (at 32 44.8) (size 0.55) (drill 0.3) (layers "F.Cu" "B.Cu") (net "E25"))
 (segment (start 32.799999 44.8) (end 38.8 42.4) (width 0.1) (layer "B.Cu") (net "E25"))
 (segment (start 32 44.8) (end 32.799999 44.8) (width 0.1) (layer "B.Cu") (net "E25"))
 (segment (start 38.8 42.4) (end 119.1 42.4) (width 0.1) (layer "B.Cu") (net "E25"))
 (segment (start 22.7625 42.7) (end 21.7 42.7) (width 0.1) (layer "F.Cu") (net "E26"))
 (via (at 21.7 42.7) (size 0.55) (drill 0.3) (layers "F.Cu" "B.Cu") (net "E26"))
 (segment (start 32.799999 45.4) (end 38.8 42.7) (width 0.1) (layer "B.Cu") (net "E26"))
 (segment (start 38.8 42.7) (end 118 42.7) (width 0.1) (layer "B.Cu") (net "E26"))
 (segment (start 26.5 42.7) (end 31.5 45.4) (width 0.1) (layer "B.Cu") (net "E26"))
 (segment (start 31.5 45.4) (end 32.799999 45.4) (width 0.1) (layer "B.Cu") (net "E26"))
 (segment (start 21.7 42.7) (end 26.5 42.7) (width 0.1) (layer "B.Cu") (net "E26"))
 (segment (start 26.5 43) (end 31.5 46) (width 0.1) (layer "F.Cu") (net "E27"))
 (segment (start 31.5 46) (end 32 46) (width 0.1) (layer "F.Cu") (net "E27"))
 (segment (start 25.6375 43) (end 26.5 43) (width 0.1) (layer "F.Cu") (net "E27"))
 (via (at 32 46) (size 0.55) (drill 0.3) (layers "F.Cu" "B.Cu") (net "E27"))
 (segment (start 38.8 43) (end 119.1 43) (width 0.1) (layer "B.Cu") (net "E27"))
 (segment (start 32.799999 46) (end 38.8 43) (width 0.1) (layer "B.Cu") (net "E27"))
 (segment (start 32 46) (end 32.799999 46) (width 0.1) (layer "B.Cu") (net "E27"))
 (segment (start 22.7625 43.3) (end 20.8 43.3) (width 0.1) (layer "F.Cu") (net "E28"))
 (via (at 20.8 43.3) (size 0.55) (drill 0.3) (layers "F.Cu" "B.Cu") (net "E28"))
 (segment (start 38.8 43.3) (end 118 43.3) (width 0.1) (layer "B.Cu") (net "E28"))
 (segment (start 20.8 43.3) (end 26.5 43.3) (width 0.1) (layer "B.Cu") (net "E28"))
 (segment (start 26.5 43.3) (end 31.5 46.6) (width 0.1) (layer "B.Cu") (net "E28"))
 (segment (start 32.799999 46.6) (end 38.8 43.3) (width 0.1) (layer "B.Cu") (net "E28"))
 (segment (start 31.5 46.6) (end 32.799999 46.6) (width 0.1) (layer "B.Cu") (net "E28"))
 (segment (start 26.5 43.6) (end 31.5 47.2) (width 0.1) (layer "F.Cu") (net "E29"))
 (segment (start 25.6375 43.6) (end 26.5 43.6) (width 0.1) (layer "F.Cu") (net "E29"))
 (segment (start 31.5 47.2) (end 32 47.2) (width 0.1) (layer "F.Cu") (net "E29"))
 (via (at 32 47.2) (size 0.55) (drill 0.3) (layers "F.Cu" "B.Cu") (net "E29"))
 (segment (start 32.799999 47.2) (end 38.8 43.6) (width 0.1) (layer "B.Cu") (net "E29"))
 (segment (start 38.8 43.6) (end 119.1 43.6) (width 0.1) (layer "B.Cu") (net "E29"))
 (segment (start 32 47.2) (end 32.799999 47.2) (width 0.1) (layer "B.Cu") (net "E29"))
 (segment (start 22.7625 43.9) (end 21.7 43.9) (width 0.1) (layer "F.Cu") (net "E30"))
 (via (at 21.7 43.9) (size 0.55) (drill 0.3) (layers "F.Cu" "B.Cu") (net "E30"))
 (segment (start 38.8 43.9) (end 118 43.9) (width 0.1) (layer "B.Cu") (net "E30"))
 (segment (start 32.799999 47.8) (end 38.8 43.9) (width 0.1) (layer "B.Cu") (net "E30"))
 (segment (start 26.5 43.9) (end 31.5 47.8) (width 0.1) (layer "B.Cu") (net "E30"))
 (segment (start 21.7 43.9) (end 26.5 43.9) (width 0.1) (layer "B.Cu") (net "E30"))
 (segment (start 31.5 47.8) (end 32.799999 47.8) (width 0.1) (layer "B.Cu") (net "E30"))
 (segment (start 26.5 44.2) (end 31.5 48.4) (width 0.1) (layer "F.Cu") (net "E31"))
 (segment (start 31.5 48.4) (end 32 48.4) (width 0.1) (layer "F.Cu") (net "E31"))
 (segment (start 25.6375 44.2) (end 26.5 44.2) (width 0.1) (layer "F.Cu") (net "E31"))
 (via (at 32 48.4) (size 0.55) (drill 0.3) (layers "F.Cu" "B.Cu") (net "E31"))
 (segment (start 32.799999 48.4) (end 38.8 44.2) (width 0.1) (layer "B.Cu") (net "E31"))
 (segment (start 38.8 44.2) (end 119.1 44.2) (width 0.1) (layer "B.Cu") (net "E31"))
 (segment (start 32 48.4) (end 32.799999 48.4) (width 0.1) (layer "B.Cu") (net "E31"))
 (segment (start 22.7625 44.5) (end 20.8 44.5) (width 0.1) (layer "F.Cu") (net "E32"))
 (via (at 20.8 44.5) (size 0.55) (drill 0.3) (layers "F.Cu" "B.Cu") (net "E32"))
 (segment (start 20.8 44.5) (end 26.5 44.5) (width 0.1) (layer "B.Cu") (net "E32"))
 (segment (start 32.799999 49) (end 38.8 44.5) (width 0.1) (layer "B.Cu") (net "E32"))
 (segment (start 26.5 44.5) (end 31.5 49) (width 0.1) (layer "B.Cu") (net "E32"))
 (segment (start 31.5 49) (end 32.799999 49) (width 0.1) (layer "B.Cu") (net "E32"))
 (segment (start 38.8 44.5) (end 118 44.5) (width 0.1) (layer "B.Cu") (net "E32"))
 (segment (start 25.6375 44.8) (end 26.5 44.8) (width 0.1) (layer "F.Cu") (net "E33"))
 (segment (start 31.5 49.6) (end 32 49.6) (width 0.1) (layer "F.Cu") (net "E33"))
 (segment (start 26.5 44.8) (end 31.5 49.6) (width 0.1) (layer "F.Cu") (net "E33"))
 (via (at 32 49.6) (size 0.55) (drill 0.3) (layers "F.Cu" "B.Cu") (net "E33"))
 (segment (start 38.8 44.8) (end 119.1 44.8) (width 0.1) (layer "B.Cu") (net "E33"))
 (segment (start 32.799999 49.6) (end 38.8 44.8) (width 0.1) (layer "B.Cu") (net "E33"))
 (segment (start 32 49.6) (end 32.799999 49.6) (width 0.1) (layer "B.Cu") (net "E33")))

